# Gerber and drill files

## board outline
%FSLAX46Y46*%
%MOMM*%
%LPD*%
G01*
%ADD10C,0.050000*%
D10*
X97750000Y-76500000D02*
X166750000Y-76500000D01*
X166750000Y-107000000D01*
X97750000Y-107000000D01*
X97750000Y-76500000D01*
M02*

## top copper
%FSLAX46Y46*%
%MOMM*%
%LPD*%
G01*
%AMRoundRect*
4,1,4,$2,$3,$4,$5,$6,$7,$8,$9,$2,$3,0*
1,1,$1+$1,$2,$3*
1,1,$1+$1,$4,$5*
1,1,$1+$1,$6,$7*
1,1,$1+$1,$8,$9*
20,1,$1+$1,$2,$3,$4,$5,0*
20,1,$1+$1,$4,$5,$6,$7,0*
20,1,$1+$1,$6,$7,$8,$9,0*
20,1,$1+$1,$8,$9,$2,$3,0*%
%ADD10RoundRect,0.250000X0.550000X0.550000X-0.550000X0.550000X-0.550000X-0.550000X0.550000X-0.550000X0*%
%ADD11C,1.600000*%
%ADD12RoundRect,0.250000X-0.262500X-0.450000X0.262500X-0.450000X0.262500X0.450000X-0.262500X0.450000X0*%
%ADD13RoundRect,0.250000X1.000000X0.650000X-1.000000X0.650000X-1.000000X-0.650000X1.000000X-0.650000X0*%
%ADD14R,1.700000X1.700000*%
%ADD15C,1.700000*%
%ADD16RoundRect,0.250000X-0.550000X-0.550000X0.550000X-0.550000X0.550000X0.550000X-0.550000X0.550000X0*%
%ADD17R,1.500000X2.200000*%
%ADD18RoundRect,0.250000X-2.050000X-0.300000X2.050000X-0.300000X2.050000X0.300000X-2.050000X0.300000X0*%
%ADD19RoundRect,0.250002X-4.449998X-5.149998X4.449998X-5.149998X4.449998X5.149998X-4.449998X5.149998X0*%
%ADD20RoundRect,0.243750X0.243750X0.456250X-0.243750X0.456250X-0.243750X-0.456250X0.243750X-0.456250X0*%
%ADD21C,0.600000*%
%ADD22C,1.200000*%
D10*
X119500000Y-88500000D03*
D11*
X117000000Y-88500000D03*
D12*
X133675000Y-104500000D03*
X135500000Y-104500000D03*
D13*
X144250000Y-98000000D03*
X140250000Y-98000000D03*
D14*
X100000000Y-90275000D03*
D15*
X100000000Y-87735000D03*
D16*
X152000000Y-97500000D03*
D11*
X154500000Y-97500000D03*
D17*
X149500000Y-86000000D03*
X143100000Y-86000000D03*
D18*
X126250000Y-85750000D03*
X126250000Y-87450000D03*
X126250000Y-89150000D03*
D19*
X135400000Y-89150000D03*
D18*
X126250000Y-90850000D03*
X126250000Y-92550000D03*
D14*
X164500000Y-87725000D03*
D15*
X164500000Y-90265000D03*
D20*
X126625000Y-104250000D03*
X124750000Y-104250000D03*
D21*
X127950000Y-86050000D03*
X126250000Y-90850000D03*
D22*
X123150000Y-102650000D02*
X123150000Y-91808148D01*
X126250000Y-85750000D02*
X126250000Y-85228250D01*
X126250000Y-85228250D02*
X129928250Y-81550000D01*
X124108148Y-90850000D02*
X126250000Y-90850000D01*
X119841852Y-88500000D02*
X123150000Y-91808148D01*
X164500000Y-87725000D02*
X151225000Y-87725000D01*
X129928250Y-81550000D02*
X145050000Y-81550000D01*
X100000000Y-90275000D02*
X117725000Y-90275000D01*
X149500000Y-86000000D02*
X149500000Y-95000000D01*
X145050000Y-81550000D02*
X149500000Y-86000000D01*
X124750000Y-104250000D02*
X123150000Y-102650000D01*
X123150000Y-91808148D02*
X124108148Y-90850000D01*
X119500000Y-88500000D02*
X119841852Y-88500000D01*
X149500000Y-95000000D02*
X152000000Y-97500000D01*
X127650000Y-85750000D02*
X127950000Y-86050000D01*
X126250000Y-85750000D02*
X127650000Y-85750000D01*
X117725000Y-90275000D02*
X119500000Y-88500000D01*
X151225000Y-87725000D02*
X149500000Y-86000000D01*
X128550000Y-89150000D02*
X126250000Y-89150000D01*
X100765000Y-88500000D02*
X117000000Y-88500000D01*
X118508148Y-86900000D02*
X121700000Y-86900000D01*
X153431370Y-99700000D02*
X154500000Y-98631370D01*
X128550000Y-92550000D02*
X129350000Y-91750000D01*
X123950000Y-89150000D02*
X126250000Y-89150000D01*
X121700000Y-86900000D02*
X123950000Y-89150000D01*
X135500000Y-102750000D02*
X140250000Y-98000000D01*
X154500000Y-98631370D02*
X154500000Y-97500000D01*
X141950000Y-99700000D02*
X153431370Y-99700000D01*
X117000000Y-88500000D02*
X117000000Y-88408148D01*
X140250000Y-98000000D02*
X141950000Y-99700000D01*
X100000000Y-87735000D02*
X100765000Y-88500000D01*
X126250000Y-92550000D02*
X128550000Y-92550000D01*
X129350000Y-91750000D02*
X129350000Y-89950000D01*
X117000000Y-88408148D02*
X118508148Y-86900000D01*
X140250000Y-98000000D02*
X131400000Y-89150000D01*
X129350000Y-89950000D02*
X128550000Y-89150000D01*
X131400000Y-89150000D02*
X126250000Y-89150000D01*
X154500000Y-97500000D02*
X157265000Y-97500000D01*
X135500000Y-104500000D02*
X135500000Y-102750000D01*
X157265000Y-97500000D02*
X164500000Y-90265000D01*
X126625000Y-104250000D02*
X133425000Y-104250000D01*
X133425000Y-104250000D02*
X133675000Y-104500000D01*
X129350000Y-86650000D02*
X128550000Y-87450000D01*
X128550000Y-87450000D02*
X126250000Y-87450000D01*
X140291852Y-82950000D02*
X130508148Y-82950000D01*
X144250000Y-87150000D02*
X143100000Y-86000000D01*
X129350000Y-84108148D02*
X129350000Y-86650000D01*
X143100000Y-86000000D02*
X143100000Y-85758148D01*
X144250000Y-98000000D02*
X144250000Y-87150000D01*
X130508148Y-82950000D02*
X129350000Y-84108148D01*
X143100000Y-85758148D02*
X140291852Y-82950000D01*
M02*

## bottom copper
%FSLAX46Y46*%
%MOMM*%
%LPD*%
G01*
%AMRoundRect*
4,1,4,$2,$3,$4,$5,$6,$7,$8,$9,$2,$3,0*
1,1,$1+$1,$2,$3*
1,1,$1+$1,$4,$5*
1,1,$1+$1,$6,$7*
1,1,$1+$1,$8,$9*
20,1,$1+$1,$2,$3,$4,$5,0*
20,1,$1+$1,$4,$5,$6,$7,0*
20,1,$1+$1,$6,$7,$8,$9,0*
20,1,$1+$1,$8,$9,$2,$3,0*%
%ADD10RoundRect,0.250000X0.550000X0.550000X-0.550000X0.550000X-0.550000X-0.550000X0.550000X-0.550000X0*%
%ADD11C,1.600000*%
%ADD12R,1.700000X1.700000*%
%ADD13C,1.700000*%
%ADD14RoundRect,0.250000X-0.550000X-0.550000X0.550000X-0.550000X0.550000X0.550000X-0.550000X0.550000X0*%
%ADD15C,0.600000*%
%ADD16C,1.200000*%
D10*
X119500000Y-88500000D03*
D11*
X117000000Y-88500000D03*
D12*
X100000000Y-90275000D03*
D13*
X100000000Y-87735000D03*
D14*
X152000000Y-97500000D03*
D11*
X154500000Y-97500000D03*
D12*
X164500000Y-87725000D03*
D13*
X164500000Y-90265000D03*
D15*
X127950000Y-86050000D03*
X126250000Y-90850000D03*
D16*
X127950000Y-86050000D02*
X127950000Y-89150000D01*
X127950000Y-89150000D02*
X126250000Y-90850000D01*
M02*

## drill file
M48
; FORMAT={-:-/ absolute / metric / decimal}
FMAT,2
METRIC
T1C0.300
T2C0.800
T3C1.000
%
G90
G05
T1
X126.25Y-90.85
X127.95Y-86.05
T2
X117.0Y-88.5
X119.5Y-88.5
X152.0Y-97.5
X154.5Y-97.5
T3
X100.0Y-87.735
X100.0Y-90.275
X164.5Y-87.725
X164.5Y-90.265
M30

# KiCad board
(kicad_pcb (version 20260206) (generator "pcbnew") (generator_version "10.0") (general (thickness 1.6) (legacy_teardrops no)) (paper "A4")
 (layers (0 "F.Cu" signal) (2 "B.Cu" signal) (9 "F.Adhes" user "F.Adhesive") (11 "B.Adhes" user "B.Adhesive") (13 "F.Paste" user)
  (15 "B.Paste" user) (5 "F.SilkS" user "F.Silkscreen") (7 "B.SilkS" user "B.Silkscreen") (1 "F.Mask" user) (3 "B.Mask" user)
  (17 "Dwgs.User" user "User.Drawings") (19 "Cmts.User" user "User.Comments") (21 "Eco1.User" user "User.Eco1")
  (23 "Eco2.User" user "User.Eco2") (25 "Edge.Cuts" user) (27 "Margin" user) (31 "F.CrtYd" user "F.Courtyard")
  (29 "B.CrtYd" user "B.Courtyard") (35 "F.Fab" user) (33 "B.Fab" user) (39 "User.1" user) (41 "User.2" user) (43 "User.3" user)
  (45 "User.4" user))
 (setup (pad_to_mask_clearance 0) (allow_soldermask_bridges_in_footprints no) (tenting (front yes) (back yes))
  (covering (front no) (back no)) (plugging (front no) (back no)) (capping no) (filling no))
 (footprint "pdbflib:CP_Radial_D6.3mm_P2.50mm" (layer "F.Cu") (at 119.5 88.5 180)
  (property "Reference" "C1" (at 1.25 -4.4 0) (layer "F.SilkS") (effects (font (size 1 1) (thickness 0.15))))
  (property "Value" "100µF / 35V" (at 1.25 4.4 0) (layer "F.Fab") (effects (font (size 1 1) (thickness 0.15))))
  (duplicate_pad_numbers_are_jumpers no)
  (pad "1" thru_hole roundrect (at 0 0 180) (size 1.6 1.6) (drill 0.8) (layers "*.Cu" "*.Mask") (remove_unused_layers no)
   (roundrect_rratio 0.15625) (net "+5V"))
  (pad "2" thru_hole circle (at 2.5 0 180) (size 1.6 1.6) (drill 0.8) (layers "*.Cu" "*.Mask") (remove_unused_layers no) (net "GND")))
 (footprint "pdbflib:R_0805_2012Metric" (layer "F.Cu") (at 134.5875 104.5)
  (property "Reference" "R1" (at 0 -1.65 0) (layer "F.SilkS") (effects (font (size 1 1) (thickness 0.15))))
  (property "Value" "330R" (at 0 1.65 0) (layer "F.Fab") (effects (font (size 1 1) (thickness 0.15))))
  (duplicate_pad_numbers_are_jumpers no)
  (pad "1" smd roundrect (at -0.9125 0) (size 1.025 1.4) (layers "F.Cu" "F.Mask" "F.Paste") (roundrect_rratio 0.243902) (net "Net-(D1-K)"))
  (pad "2" smd roundrect (at 0.9125 0) (size 1.025 1.4) (layers "F.Cu" "F.Mask" "F.Paste") (roundrect_rratio 0.243902) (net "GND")))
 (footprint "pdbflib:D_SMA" (layer "F.Cu") (at 142.25 98 180)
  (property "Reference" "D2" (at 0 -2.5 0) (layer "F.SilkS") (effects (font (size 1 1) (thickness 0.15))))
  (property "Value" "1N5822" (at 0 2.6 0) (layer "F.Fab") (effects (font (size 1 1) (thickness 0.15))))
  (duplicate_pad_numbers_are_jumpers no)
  (pad "1" smd roundrect (at -2 0 180) (size 2.5 1.8) (layers "F.Cu" "F.Mask" "F.Paste") (roundrect_rratio 0.1388888889) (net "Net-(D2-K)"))
  (pad "2" smd roundrect (at 2 0 180) (size 2.5 1.8) (layers "F.Cu" "F.Mask" "F.Paste") (roundrect_rratio 0.1388888889) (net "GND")))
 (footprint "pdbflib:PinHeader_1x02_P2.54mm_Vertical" (layer "F.Cu") (at 100 90.275 180)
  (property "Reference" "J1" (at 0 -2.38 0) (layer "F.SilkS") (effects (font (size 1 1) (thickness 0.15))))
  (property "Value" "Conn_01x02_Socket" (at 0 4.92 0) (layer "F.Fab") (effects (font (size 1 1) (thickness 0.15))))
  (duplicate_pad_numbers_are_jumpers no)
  (pad "1" thru_hole rect (at 0 0 180) (size 1.7 1.7) (drill 1) (layers "*.Cu" "*.Mask") (remove_unused_layers no) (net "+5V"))
  (pad "2" thru_hole circle (at 0 2.54 180) (size 1.7 1.7) (drill 1) (layers "*.Cu" "*.Mask") (remove_unused_layers no) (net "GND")))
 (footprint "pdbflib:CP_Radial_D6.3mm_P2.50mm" (layer "F.Cu") (at 152 97.5)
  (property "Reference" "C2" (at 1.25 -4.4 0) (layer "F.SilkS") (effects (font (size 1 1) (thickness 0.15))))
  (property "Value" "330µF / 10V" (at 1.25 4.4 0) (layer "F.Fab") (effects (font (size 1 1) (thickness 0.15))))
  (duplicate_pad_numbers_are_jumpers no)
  (pad "1" thru_hole roundrect (at 0 0) (size 1.6 1.6) (drill 0.8) (layers "*.Cu" "*.Mask") (remove_unused_layers no)
   (roundrect_rratio 0.15625) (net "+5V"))
  (pad "2" thru_hole circle (at 2.5 0) (size 1.6 1.6) (drill 0.8) (layers "*.Cu" "*.Mask") (remove_unused_layers no) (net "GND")))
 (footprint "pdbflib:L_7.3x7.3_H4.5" (layer "F.Cu") (at 146.3 86 180)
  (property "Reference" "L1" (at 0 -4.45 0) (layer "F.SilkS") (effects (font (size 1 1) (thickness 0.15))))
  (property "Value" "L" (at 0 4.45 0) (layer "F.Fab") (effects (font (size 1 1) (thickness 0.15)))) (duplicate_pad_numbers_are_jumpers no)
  (pad "1" smd rect (at -3.2 0 180) (size 1.5 2.2) (layers "F.Cu" "F.Mask" "F.Paste") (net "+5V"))
  (pad "2" smd rect (at 3.2 0 180) (size 1.5 2.2) (layers "F.Cu" "F.Mask" "F.Paste") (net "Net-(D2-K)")))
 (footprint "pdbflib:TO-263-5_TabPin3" (layer "F.Cu") (at 133.9 89.15)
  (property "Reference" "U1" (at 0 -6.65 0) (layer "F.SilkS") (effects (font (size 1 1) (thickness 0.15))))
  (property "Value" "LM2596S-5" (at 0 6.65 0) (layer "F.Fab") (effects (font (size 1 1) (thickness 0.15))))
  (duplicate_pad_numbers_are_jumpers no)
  (pad "" smd roundrect (at -0.925 -2.775) (size 4.55 5.25) (layers "F.Paste") (roundrect_rratio 0.054945))
  (pad "" smd roundrect (at -0.925 2.775) (size 4.55 5.25) (layers "F.Paste") (roundrect_rratio 0.054945))
  (pad "" smd roundrect (at 3.925 -2.775) (size 4.55 5.25) (layers "F.Paste") (roundrect_rratio 0.054945))
  (pad "" smd roundrect (at 3.925 2.775) (size 4.55 5.25) (layers "F.Paste") (roundrect_rratio 0.054945))
  (pad "1" smd roundrect (at -7.65 -3.4) (size 4.6 1.1) (layers "F.Cu" "F.Mask" "F.Paste") (roundrect_rratio 0.227273) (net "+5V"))
  (pad "2" smd roundrect (at -7.65 -1.7) (size 4.6 1.1) (layers "F.Cu" "F.Mask" "F.Paste") (roundrect_rratio 0.227273) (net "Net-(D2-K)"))
  (pad "3" smd roundrect (at -7.65 0) (size 4.6 1.1) (layers "F.Cu" "F.Mask" "F.Paste") (roundrect_rratio 0.227273) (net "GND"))
  (pad "3" smd roundrect (at 1.5 0) (size 9.4 10.8) (layers "F.Cu" "F.Mask") (roundrect_rratio 0.026596) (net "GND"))
  (pad "4" smd roundrect (at -7.65 1.7) (size 4.6 1.1) (layers "F.Cu" "F.Mask" "F.Paste") (roundrect_rratio 0.227273) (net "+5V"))
  (pad "5" smd roundrect (at -7.65 3.4) (size 4.6 1.1) (layers "F.Cu" "F.Mask" "F.Paste") (roundrect_rratio 0.227273) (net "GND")))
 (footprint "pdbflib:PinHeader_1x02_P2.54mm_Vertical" (layer "F.Cu") (at 164.5 87.725)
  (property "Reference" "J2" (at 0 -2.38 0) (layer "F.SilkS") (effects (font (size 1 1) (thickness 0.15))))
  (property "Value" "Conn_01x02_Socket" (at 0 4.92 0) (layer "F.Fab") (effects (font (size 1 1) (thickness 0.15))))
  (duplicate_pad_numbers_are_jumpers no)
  (pad "1" thru_hole rect (at 0 0) (size 1.7 1.7) (drill 1) (layers "*.Cu" "*.Mask") (remove_unused_layers no) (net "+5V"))
  (pad "2" thru_hole circle (at 0 2.54) (size 1.7 1.7) (drill 1) (layers "*.Cu" "*.Mask") (remove_unused_layers no) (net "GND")))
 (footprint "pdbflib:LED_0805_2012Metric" (layer "F.Cu") (at 125.6875 104.25 180)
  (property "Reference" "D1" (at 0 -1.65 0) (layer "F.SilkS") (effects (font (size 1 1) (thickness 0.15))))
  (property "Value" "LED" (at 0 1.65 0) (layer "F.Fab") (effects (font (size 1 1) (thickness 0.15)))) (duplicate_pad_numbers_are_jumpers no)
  (pad "1" smd roundrect (at -0.9375 0 180) (size 0.975 1.4) (layers "F.Cu" "F.Mask" "F.Paste") (roundrect_rratio 0.25) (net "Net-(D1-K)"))
  (pad "2" smd roundrect (at 0.9375 0 180) (size 0.975 1.4) (layers "F.Cu" "F.Mask" "F.Paste") (roundrect_rratio 0.25) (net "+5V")))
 (gr_rect (start 97.75 76.5) (end 166.75 107) (stroke (width 0.05) (type default)) (fill no) (layer "Edge.Cuts"))
 (segment (start 123.15 102.65) (end 123.15 91.808148) (width 1.2) (layer "F.Cu") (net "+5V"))
 (segment (start 126.25 85.75) (end 126.25 85.22825) (width 1.2) (layer "F.Cu") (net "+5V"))
 (segment (start 126.25 85.22825) (end 129.92825 81.55) (width 1.2) (layer "F.Cu") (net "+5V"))
 (segment (start 124.108148 90.85) (end 126.25 90.85) (width 1.2) (layer "F.Cu") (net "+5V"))
 (segment (start 119.841852 88.5) (end 123.15 91.808148) (width 1.2) (layer "F.Cu") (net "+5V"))
 (segment (start 164.5 87.725) (end 151.225 87.725) (width 1.2) (layer "F.Cu") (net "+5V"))
 (segment (start 129.92825 81.55) (end 145.05 81.55) (width 1.2) (layer "F.Cu") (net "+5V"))
 (segment (start 100 90.275) (end 117.725 90.275) (width 1.2) (layer "F.Cu") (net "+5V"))
 (segment (start 149.5 86) (end 149.5 95) (width 1.2) (layer "F.Cu") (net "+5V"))
 (segment (start 145.05 81.55) (end 149.5 86) (width 1.2) (layer "F.Cu") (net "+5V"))
 (segment (start 124.75 104.25) (end 123.15 102.65) (width 1.2) (layer "F.Cu") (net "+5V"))
 (segment (start 123.15 91.808148) (end 124.108148 90.85) (width 1.2) (layer "F.Cu") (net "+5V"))
 (segment (start 119.5 88.5) (end 119.841852 88.5) (width 1.2) (layer "F.Cu") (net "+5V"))
 (segment (start 149.5 95) (end 152 97.5) (width 1.2) (layer "F.Cu") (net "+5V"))
 (segment (start 127.65 85.75) (end 127.95 86.05) (width 1.2) (layer "F.Cu") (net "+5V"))
 (segment (start 126.25 85.75) (end 127.65 85.75) (width 1.2) (layer "F.Cu") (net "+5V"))
 (segment (start 117.725 90.275) (end 119.5 88.5) (width 1.2) (layer "F.Cu") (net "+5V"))
 (segment (start 151.225 87.725) (end 149.5 86) (width 1.2) (layer "F.Cu") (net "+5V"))
 (via (at 127.95 86.05) (size 0.6) (drill 0.3) (layers "F.Cu" "B.Cu") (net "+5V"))
 (via (at 126.25 90.85) (size 0.6) (drill 0.3) (layers "F.Cu" "B.Cu") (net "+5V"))
 (segment (start 127.95 86.05) (end 127.95 89.15) (width 1.2) (layer "B.Cu") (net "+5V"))
 (segment (start 127.95 89.15) (end 126.25 90.85) (width 1.2) (layer "B.Cu") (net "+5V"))
 (segment (start 128.55 89.15) (end 126.25 89.15) (width 1.2) (layer "F.Cu") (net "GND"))
 (segment (start 100.765 88.5) (end 117 88.5) (width 1.2) (layer "F.Cu") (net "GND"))
 (segment (start 118.508148 86.9) (end 121.7 86.9) (width 1.2) (layer "F.Cu") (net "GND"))
 (segment (start 153.43137 99.7) (end 154.5 98.63137) (width 1.2) (layer "F.Cu") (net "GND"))
 (segment (start 128.55 92.55) (end 129.35 91.75) (width 1.2) (layer "F.Cu") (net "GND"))
 (segment (start 123.95 89.15) (end 126.25 89.15) (width 1.2) (layer "F.Cu") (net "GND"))
 (segment (start 121.7 86.9) (end 123.95 89.15) (width 1.2) (layer "F.Cu") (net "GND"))
 (segment (start 135.5 102.75) (end 140.25 98) (width 1.2) (layer "F.Cu") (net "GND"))
 (segment (start 154.5 98.63137) (end 154.5 97.5) (width 1.2) (layer "F.Cu") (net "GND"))
 (segment (start 141.95 99.7) (end 153.43137 99.7) (width 1.2) (layer "F.Cu") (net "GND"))
 (segment (start 117 88.5) (end 117 88.408148) (width 1.2) (layer "F.Cu") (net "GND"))
 (segment (start 140.25 98) (end 141.95 99.7) (width 1.2) (layer "F.Cu") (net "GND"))
 (segment (start 100 87.735) (end 100.765 88.5) (width 1.2) (layer "F.Cu") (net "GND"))
 (segment (start 126.25 92.55) (end 128.55 92.55) (width 1.2) (layer "F.Cu") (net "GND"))
 (segment (start 129.35 91.75) (end 129.35 89.95) (width 1.2) (layer "F.Cu") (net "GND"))
 (segment (start 117 88.408148) (end 118.508148 86.9) (width 1.2) (layer "F.Cu") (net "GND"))
 (segment (start 140.25 98) (end 131.4 89.15) (width 1.2) (layer "F.Cu") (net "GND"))
 (segment (start 129.35 89.95) (end 128.55 89.15) (width 1.2) (layer "F.Cu") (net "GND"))
 (segment (start 131.4 89.15) (end 126.25 89.15) (width 1.2) (layer "F.Cu") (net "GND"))
 (segment (start 154.5 97.5) (end 157.265 97.5) (width 1.2) (layer "F.Cu") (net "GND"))
 (segment (start 135.5 104.5) (end 135.5 102.75) (width 1.2) (layer "F.Cu") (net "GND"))
 (segment (start 157.265 97.5) (end 164.5 90.265) (width 1.2) (layer "F.Cu") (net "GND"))
 (segment (start 126.625 104.25) (end 133.425 104.25) (width 1.2) (layer "F.Cu") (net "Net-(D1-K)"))
 (segment (start 133.425 104.25) (end 133.675 104.5) (width 1.2) (layer "F.Cu") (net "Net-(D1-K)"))
 (segment (start 129.35 86.65) (end 128.55 87.45) (width 1.2) (layer "F.Cu") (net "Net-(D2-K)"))
 (segment (start 128.55 87.45) (end 126.25 87.45) (width 1.2) (layer "F.Cu") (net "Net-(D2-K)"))
 (segment (start 140.291852 82.95) (end 130.508148 82.95) (width 1.2) (layer "F.Cu") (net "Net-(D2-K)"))
 (segment (start 144.25 87.15) (end 143.1 86) (width 1.2) (layer "F.Cu") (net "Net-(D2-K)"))
 (segment (start 129.35 84.108148) (end 129.35 86.65) (width 1.2) (layer "F.Cu") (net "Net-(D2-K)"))
 (segment (start 143.1 86) (end 143.1 85.758148) (width 1.2) (layer "F.Cu") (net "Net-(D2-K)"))
 (segment (start 144.25 98) (end 144.25 87.15) (width 1.2) (layer "F.Cu") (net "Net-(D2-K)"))
 (segment (start 130.508148 82.95) (end 129.35 84.108148) (width 1.2) (layer "F.Cu") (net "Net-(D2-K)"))
 (segment (start 143.1 85.758148) (end 140.291852 82.95) (width 1.2) (layer "F.Cu") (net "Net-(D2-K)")))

